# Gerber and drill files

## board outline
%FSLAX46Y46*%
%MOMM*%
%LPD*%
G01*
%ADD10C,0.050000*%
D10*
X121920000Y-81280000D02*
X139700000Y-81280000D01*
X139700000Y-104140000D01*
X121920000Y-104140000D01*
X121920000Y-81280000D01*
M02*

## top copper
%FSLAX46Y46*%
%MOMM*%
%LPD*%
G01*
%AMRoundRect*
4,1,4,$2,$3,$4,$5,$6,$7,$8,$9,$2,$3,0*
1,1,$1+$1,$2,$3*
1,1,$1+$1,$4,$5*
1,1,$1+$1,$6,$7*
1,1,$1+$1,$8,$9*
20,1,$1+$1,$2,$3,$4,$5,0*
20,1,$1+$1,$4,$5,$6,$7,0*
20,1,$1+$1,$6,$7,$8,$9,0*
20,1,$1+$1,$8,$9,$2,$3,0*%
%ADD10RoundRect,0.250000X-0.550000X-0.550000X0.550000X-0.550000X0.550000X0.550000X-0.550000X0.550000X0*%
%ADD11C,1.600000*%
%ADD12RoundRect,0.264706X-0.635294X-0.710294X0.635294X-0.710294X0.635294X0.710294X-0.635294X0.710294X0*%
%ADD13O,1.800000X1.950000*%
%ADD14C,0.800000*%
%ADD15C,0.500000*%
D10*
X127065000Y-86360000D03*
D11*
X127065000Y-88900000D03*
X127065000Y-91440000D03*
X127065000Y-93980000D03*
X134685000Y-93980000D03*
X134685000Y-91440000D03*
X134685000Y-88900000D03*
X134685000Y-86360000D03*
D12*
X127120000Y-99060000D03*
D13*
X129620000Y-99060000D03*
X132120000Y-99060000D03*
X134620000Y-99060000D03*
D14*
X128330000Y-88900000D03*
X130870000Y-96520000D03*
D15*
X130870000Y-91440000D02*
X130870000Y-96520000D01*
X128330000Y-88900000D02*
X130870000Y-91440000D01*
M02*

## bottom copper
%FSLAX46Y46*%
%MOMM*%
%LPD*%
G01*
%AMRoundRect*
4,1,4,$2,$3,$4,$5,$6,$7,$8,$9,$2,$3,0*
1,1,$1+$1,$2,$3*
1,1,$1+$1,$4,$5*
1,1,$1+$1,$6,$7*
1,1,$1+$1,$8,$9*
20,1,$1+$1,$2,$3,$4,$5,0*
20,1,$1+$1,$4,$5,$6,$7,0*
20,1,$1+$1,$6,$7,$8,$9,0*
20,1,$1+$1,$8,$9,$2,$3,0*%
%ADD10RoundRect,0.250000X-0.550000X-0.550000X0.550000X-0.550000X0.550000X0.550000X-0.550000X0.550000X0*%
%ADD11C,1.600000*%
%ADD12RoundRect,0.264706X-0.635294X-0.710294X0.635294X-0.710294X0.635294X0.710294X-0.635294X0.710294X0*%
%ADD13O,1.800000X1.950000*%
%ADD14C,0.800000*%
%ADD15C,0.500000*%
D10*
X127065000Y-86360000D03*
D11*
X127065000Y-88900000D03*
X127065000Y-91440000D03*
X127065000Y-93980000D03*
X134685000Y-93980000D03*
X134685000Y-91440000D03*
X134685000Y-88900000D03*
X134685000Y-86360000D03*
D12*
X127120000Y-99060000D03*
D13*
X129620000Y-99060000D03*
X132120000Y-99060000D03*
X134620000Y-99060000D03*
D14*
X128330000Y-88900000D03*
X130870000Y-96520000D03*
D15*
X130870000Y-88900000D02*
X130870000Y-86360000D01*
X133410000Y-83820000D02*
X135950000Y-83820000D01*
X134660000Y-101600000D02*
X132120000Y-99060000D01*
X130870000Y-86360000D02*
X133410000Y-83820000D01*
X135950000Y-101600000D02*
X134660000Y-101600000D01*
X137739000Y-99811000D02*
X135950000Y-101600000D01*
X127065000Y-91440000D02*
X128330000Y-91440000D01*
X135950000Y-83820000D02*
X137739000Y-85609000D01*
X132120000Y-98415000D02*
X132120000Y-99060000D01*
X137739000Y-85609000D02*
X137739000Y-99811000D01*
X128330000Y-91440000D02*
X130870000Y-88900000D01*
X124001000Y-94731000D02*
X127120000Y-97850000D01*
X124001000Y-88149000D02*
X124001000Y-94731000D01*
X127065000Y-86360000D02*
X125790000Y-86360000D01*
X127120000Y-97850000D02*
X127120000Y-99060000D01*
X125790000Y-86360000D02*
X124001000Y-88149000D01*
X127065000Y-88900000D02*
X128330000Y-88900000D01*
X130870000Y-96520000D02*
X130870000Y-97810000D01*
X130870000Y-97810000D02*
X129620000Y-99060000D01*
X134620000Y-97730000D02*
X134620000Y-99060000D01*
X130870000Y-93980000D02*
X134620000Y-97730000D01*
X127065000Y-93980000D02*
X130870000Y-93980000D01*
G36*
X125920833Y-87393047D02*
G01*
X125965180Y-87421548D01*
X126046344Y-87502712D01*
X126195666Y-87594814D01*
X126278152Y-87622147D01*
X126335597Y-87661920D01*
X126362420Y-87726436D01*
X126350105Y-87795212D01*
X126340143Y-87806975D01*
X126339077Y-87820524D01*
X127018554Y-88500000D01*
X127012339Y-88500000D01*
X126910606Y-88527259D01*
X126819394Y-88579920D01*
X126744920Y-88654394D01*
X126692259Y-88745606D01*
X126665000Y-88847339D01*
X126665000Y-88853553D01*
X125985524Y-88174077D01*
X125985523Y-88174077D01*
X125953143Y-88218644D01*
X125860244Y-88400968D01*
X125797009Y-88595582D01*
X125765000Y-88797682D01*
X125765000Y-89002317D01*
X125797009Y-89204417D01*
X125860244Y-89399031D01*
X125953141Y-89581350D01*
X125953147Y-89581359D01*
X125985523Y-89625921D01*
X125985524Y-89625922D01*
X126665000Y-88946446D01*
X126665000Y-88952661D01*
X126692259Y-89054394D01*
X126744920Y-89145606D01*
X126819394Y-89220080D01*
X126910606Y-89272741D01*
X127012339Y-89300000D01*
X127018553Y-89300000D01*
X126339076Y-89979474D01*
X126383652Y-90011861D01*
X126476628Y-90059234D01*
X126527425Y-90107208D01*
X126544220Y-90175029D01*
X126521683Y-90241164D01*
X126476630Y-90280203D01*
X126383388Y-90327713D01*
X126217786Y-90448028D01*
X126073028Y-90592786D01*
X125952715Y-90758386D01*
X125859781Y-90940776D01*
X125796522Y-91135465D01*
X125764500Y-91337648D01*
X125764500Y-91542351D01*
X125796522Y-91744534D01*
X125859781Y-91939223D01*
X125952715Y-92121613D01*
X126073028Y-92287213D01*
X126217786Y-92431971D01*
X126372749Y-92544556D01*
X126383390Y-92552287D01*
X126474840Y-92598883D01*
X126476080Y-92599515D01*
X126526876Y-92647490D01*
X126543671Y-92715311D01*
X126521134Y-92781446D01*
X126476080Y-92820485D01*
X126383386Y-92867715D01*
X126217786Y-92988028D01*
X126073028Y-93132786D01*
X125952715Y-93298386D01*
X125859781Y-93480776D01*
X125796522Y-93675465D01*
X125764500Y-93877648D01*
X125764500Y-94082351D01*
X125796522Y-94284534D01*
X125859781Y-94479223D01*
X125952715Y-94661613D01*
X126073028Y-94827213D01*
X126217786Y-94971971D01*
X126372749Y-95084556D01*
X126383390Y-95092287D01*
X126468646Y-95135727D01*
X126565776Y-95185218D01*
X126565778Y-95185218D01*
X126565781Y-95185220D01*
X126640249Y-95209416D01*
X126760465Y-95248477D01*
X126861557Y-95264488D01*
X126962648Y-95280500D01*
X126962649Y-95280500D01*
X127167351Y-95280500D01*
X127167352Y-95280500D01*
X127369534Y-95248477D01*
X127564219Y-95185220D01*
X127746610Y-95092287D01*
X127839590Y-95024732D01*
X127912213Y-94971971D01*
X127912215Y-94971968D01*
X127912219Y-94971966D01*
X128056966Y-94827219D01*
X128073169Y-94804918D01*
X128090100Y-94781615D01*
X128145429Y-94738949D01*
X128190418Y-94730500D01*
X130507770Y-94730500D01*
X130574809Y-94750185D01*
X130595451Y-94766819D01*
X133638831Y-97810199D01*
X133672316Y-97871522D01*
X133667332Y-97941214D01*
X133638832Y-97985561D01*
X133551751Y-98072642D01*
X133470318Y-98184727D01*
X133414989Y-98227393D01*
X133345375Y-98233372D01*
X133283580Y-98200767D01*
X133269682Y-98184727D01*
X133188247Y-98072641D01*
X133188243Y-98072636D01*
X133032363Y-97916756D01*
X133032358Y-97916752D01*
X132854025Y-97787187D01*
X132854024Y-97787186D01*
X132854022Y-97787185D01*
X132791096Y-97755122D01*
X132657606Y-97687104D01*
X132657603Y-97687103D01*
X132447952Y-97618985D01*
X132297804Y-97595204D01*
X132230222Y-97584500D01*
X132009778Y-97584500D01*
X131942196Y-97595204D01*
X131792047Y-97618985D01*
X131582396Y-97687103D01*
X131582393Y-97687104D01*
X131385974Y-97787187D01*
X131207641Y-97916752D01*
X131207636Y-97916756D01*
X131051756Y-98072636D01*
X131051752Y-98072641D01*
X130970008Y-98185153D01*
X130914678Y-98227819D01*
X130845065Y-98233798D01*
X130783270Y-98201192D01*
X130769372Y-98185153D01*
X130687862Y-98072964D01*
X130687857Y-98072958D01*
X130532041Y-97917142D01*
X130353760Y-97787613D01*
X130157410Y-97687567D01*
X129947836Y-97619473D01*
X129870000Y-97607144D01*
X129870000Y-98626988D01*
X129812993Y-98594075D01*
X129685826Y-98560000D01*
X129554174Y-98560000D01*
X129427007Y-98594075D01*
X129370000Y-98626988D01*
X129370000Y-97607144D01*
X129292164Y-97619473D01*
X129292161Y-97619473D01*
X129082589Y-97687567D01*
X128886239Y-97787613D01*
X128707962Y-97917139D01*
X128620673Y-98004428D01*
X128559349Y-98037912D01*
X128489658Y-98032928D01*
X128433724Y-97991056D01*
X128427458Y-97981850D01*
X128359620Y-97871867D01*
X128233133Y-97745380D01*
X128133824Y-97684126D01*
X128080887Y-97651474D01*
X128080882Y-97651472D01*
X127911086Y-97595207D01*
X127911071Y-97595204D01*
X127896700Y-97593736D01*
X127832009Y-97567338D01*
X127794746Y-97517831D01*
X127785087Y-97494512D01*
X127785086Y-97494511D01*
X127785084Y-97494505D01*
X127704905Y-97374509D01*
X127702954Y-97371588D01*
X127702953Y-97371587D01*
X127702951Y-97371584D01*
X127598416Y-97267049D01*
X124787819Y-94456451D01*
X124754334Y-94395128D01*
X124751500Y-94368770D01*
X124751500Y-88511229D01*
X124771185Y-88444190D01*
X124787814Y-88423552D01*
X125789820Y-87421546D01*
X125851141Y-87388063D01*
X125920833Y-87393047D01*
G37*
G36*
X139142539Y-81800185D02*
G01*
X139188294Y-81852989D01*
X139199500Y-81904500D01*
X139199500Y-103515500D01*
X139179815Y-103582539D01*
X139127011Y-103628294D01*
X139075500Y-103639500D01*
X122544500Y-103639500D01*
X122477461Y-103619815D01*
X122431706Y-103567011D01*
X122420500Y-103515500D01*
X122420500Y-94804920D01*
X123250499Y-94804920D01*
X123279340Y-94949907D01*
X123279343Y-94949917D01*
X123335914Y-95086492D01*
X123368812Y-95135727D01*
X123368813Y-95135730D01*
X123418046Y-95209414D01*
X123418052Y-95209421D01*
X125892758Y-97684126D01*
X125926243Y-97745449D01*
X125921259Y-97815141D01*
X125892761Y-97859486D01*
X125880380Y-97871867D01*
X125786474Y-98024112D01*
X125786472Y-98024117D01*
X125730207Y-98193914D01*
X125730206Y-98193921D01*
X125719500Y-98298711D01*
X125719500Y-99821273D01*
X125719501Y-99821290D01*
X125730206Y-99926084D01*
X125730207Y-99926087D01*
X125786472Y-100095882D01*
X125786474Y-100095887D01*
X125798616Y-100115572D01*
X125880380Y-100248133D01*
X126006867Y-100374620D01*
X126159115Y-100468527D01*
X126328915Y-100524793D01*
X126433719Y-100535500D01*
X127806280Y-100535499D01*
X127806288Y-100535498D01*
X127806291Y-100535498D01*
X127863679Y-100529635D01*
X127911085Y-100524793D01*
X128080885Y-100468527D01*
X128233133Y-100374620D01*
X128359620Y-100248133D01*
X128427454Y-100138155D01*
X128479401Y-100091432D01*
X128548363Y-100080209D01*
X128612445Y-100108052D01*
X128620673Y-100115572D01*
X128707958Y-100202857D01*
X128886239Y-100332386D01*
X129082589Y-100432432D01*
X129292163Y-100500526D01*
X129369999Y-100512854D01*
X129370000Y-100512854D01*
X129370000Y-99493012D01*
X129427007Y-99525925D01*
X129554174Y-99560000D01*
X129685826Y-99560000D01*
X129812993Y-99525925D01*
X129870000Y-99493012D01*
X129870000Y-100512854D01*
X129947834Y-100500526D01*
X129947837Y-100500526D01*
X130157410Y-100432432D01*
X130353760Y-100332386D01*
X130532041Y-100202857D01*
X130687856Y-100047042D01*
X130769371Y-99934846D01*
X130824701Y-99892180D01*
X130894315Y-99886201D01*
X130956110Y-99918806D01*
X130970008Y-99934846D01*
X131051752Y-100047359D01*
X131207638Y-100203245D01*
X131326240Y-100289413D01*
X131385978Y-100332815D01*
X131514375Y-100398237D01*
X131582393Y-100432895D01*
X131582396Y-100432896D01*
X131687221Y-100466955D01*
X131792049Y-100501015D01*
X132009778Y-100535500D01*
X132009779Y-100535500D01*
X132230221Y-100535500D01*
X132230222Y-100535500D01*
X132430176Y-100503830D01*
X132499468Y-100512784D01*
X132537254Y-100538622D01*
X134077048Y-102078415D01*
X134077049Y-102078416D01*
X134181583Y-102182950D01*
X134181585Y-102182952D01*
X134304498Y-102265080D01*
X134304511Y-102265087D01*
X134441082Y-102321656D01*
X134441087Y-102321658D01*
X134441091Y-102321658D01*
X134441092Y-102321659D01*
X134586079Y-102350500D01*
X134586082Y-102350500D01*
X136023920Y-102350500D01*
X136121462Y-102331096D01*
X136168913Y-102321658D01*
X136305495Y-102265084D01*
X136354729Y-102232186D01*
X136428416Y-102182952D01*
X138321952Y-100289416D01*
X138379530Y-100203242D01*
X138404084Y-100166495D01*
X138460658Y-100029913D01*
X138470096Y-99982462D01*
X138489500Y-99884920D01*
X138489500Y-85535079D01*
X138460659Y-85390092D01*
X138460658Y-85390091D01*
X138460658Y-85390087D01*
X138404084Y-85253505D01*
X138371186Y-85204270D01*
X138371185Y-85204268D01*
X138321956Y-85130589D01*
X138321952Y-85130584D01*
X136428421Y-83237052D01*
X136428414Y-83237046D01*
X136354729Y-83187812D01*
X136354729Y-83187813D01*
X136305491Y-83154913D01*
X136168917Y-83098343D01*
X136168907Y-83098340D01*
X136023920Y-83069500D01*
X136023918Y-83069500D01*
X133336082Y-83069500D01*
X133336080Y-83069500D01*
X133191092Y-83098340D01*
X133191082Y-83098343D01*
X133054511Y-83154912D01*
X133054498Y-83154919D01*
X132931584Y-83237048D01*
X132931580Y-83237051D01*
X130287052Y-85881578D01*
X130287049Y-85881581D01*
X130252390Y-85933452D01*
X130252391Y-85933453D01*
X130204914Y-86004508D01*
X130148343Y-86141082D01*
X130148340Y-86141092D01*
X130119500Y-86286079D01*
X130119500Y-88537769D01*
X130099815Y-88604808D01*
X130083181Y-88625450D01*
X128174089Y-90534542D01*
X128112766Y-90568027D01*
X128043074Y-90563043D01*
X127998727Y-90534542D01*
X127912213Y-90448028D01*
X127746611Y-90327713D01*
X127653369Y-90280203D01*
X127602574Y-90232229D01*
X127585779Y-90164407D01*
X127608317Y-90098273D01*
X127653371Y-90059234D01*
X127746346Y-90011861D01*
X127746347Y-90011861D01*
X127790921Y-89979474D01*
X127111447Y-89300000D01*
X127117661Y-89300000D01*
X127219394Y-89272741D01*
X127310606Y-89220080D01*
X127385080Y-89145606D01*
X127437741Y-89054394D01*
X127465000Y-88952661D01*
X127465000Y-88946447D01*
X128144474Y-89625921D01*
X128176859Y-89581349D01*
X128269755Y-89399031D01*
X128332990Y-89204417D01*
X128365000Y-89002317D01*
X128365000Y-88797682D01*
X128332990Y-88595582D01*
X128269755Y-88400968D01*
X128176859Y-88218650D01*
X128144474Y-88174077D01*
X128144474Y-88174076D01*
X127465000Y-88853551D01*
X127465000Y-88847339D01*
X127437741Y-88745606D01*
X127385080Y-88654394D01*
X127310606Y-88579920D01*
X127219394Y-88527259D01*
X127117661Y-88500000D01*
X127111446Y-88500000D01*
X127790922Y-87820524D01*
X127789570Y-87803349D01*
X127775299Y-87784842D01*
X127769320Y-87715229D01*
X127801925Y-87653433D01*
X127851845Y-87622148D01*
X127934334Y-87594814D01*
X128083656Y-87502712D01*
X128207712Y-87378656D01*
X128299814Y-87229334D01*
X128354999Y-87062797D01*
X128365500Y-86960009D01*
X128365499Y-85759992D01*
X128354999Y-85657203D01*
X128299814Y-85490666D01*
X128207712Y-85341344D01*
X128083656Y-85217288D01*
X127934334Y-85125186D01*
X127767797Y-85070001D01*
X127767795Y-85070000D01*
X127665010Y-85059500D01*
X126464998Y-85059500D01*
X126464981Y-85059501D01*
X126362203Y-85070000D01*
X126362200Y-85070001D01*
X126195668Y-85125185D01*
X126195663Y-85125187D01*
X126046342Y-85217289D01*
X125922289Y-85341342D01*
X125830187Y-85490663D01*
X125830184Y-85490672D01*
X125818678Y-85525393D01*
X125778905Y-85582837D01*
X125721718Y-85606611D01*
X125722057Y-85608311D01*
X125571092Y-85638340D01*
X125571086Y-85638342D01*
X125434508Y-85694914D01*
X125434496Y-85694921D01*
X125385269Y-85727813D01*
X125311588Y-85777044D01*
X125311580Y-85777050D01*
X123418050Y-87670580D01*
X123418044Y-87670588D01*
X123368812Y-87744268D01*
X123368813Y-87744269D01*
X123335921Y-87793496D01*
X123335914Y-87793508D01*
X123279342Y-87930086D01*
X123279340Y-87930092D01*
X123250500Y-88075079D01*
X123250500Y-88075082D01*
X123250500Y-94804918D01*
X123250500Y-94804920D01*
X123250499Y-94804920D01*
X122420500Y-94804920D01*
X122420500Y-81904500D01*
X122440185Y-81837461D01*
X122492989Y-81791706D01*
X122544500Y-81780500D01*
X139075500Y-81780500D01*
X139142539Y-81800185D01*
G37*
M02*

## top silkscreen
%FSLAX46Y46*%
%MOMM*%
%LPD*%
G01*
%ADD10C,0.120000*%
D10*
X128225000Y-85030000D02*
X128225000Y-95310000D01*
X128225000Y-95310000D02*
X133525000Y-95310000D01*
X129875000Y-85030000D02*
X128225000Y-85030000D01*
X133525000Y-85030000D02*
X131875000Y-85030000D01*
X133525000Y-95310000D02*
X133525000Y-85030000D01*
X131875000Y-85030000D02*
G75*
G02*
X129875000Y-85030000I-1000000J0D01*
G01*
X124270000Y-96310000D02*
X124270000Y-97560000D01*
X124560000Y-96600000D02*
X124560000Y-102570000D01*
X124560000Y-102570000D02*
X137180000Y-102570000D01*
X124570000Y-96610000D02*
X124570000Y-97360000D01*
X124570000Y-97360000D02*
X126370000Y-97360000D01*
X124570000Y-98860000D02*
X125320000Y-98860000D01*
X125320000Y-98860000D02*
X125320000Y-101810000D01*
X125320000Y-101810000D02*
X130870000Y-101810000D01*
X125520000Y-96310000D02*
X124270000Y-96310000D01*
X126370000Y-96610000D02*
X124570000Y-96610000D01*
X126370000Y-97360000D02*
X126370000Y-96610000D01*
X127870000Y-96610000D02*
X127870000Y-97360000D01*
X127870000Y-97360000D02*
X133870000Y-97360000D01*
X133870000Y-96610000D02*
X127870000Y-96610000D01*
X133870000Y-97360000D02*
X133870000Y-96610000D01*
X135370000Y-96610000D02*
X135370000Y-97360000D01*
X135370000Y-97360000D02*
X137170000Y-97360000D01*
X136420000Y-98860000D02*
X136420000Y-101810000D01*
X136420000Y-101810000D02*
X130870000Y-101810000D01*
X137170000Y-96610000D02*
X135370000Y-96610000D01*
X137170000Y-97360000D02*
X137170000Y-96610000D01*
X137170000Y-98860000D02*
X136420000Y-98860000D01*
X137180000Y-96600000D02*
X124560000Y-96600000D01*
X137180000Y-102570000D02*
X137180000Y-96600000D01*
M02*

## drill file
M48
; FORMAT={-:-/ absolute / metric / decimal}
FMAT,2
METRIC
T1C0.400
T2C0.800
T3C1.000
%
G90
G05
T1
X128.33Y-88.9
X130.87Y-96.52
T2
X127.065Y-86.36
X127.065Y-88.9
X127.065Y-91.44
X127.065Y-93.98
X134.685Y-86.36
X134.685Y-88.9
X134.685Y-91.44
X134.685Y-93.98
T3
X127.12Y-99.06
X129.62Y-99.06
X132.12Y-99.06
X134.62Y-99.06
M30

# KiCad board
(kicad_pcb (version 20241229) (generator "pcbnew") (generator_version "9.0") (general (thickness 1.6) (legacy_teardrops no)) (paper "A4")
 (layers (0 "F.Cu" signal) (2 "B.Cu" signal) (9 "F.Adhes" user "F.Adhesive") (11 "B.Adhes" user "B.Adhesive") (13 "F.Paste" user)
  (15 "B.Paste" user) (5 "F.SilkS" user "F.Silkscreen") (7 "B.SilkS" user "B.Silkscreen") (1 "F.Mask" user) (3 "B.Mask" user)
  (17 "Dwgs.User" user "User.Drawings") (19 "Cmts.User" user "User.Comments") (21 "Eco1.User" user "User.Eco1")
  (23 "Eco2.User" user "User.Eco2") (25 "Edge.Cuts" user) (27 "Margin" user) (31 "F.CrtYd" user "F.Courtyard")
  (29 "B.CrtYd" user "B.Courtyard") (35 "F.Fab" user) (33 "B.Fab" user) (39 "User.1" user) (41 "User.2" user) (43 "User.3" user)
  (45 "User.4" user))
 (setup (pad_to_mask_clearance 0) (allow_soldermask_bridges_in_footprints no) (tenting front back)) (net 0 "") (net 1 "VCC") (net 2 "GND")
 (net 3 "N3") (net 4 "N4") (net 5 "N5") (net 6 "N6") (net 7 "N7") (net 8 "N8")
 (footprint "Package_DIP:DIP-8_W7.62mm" (layer "F.Cu") (at 127.065 86.36)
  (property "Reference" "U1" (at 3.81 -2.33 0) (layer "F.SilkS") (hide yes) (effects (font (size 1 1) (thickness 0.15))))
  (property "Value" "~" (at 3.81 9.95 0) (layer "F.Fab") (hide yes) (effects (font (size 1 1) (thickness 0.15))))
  (fp_line (start 1.16 -1.33) (end 1.16 8.95) (stroke (width 0.12) (type solid)) (layer "F.SilkS"))
  (fp_line (start 1.16 8.95) (end 6.46 8.95) (stroke (width 0.12) (type solid)) (layer "F.SilkS"))
  (fp_line (start 2.81 -1.33) (end 1.16 -1.33) (stroke (width 0.12) (type solid)) (layer "F.SilkS"))
  (fp_line (start 6.46 -1.33) (end 4.81 -1.33) (stroke (width 0.12) (type solid)) (layer "F.SilkS"))
  (fp_line (start 6.46 8.95) (end 6.46 -1.33) (stroke (width 0.12) (type solid)) (layer "F.SilkS"))
  (fp_arc (start 4.81 -1.33) (mid 3.81 -0.33) (end 2.81 -1.33) (stroke (width 0.12) (type solid)) (layer "F.SilkS"))
  (pad "1" thru_hole roundrect (at 0 0) (size 1.6 1.6) (drill 0.8) (layers "*.Cu" "*.Mask") (remove_unused_layers no)
   (roundrect_rratio 0.15625) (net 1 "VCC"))
  (pad "2" thru_hole circle (at 0 2.54) (size 1.6 1.6) (drill 0.8) (layers "*.Cu" "*.Mask") (remove_unused_layers no) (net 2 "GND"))
  (pad "3" thru_hole circle (at 0 5.08) (size 1.6 1.6) (drill 0.8) (layers "*.Cu" "*.Mask") (remove_unused_layers no) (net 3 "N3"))
  (pad "4" thru_hole circle (at 0 7.62) (size 1.6 1.6) (drill 0.8) (layers "*.Cu" "*.Mask") (remove_unused_layers no) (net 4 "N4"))
  (pad "5" thru_hole circle (at 7.62 7.62) (size 1.6 1.6) (drill 0.8) (layers "*.Cu" "*.Mask") (remove_unused_layers no) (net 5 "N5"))
  (pad "6" thru_hole circle (at 7.62 5.08) (size 1.6 1.6) (drill 0.8) (layers "*.Cu" "*.Mask") (remove_unused_layers no) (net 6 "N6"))
  (pad "7" thru_hole circle (at 7.62 2.54) (size 1.6 1.6) (drill 0.8) (layers "*.Cu" "*.Mask") (remove_unused_layers no) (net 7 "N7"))
  (pad "8" thru_hole circle (at 7.62 0) (size 1.6 1.6) (drill 0.8) (layers "*.Cu" "*.Mask") (remove_unused_layers no) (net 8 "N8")))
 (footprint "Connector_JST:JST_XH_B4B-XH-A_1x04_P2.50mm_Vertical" (layer "F.Cu") (at 127.12 99.06)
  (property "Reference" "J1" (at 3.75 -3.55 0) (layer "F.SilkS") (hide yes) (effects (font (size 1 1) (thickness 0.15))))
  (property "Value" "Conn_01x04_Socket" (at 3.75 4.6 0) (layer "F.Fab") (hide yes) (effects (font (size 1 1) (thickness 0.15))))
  (fp_line (start -2.85 -2.75) (end -2.85 -1.5) (stroke (width 0.12) (type solid)) (layer "F.SilkS"))
  (fp_line (start -2.56 -2.46) (end -2.56 3.51) (stroke (width 0.12) (type solid)) (layer "F.SilkS"))
  (fp_line (start -2.56 3.51) (end 10.06 3.51) (stroke (width 0.12) (type solid)) (layer "F.SilkS"))
  (fp_line (start -2.55 -2.45) (end -2.55 -1.7) (stroke (width 0.12) (type solid)) (layer "F.SilkS"))
  (fp_line (start -2.55 -1.7) (end -0.75 -1.7) (stroke (width 0.12) (type solid)) (layer "F.SilkS"))
  (fp_line (start -2.55 -0.2) (end -1.8 -0.2) (stroke (width 0.12) (type solid)) (layer "F.SilkS"))
  (fp_line (start -1.8 -0.2) (end -1.8 2.75) (stroke (width 0.12) (type solid)) (layer "F.SilkS"))
  (fp_line (start -1.8 2.75) (end 3.75 2.75) (stroke (width 0.12) (type solid)) (layer "F.SilkS"))
  (fp_line (start -1.6 -2.75) (end -2.85 -2.75) (stroke (width 0.12) (type solid)) (layer "F.SilkS"))
  (fp_line (start -0.75 -2.45) (end -2.55 -2.45) (stroke (width 0.12) (type solid)) (layer "F.SilkS"))
  (fp_line (start -0.75 -1.7) (end -0.75 -2.45) (stroke (width 0.12) (type solid)) (layer "F.SilkS"))
  (fp_line (start 0.75 -2.45) (end 0.75 -1.7) (stroke (width 0.12) (type solid)) (layer "F.SilkS"))
  (fp_line (start 0.75 -1.7) (end 6.75 -1.7) (stroke (width 0.12) (type solid)) (layer "F.SilkS"))
  (fp_line (start 6.75 -2.45) (end 0.75 -2.45) (stroke (width 0.12) (type solid)) (layer "F.SilkS"))
  (fp_line (start 6.75 -1.7) (end 6.75 -2.45) (stroke (width 0.12) (type solid)) (layer "F.SilkS"))
  (fp_line (start 8.25 -2.45) (end 8.25 -1.7) (stroke (width 0.12) (type solid)) (layer "F.SilkS"))
  (fp_line (start 8.25 -1.7) (end 10.05 -1.7) (stroke (width 0.12) (type solid)) (layer "F.SilkS"))
  (fp_line (start 9.3 -0.2) (end 9.3 2.75) (stroke (width 0.12) (type solid)) (layer "F.SilkS"))
  (fp_line (start 9.3 2.75) (end 3.75 2.75) (stroke (width 0.12) (type solid)) (layer "F.SilkS"))
  (fp_line (start 10.05 -2.45) (end 8.25 -2.45) (stroke (width 0.12) (type solid)) (layer "F.SilkS"))
  (fp_line (start 10.05 -1.7) (end 10.05 -2.45) (stroke (width 0.12) (type solid)) (layer "F.SilkS"))
  (fp_line (start 10.05 -0.2) (end 9.3 -0.2) (stroke (width 0.12) (type solid)) (layer "F.SilkS"))
  (fp_line (start 10.06 -2.46) (end -2.56 -2.46) (stroke (width 0.12) (type solid)) (layer "F.SilkS"))
  (fp_line (start 10.06 3.51) (end 10.06 -2.46) (stroke (width 0.12) (type solid)) (layer "F.SilkS"))
  (pad "1" thru_hole roundrect (at 0 0) (size 1.8 1.95) (drill 1) (layers "*.Cu" "*.Mask") (remove_unused_layers no)
   (roundrect_rratio 0.147059) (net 1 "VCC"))
  (pad "2" thru_hole oval (at 2.5 0) (size 1.8 1.95) (drill 1) (layers "*.Cu" "*.Mask") (remove_unused_layers no) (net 2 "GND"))
  (pad "3" thru_hole oval (at 5 0) (size 1.8 1.95) (drill 1) (layers "*.Cu" "*.Mask") (remove_unused_layers no) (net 3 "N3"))
  (pad "4" thru_hole oval (at 7.5 0) (size 1.8 1.95) (drill 1) (layers "*.Cu" "*.Mask") (remove_unused_layers no) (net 4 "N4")))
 (gr_rect (start 121.92 81.28) (end 139.7 104.14) (stroke (width 0.05) (type default)) (fill no) (layer "Edge.Cuts"))
 (segment (start 130.87 88.9) (end 130.87 86.36) (width 0.5) (layer "B.Cu") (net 3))
 (segment (start 133.41 83.82) (end 135.95 83.82) (width 0.5) (layer "B.Cu") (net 3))
 (segment (start 134.66 101.6) (end 132.12 99.06) (width 0.5) (layer "B.Cu") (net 3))
 (segment (start 130.87 86.36) (end 133.41 83.82) (width 0.5) (layer "B.Cu") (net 3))
 (segment (start 135.95 101.6) (end 134.66 101.6) (width 0.5) (layer "B.Cu") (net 3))
 (segment (start 137.739 99.811) (end 135.95 101.6) (width 0.5) (layer "B.Cu") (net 3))
 (segment (start 127.065 91.44) (end 128.33 91.44) (width 0.5) (layer "B.Cu") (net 3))
 (segment (start 135.95 83.82) (end 137.739 85.609) (width 0.5) (layer "B.Cu") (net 3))
 (segment (start 132.12 98.415) (end 132.12 99.06) (width 0.5) (layer "B.Cu") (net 3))
 (segment (start 137.739 85.609) (end 137.739 99.811) (width 0.5) (layer "B.Cu") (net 3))
 (segment (start 128.33 91.44) (end 130.87 88.9) (width 0.5) (layer "B.Cu") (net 3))
 (segment (start 124.001 94.731) (end 127.12 97.85) (width 0.5) (layer "B.Cu") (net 1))
 (segment (start 124.001 88.149) (end 124.001 94.731) (width 0.5) (layer "B.Cu") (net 1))
 (segment (start 127.065 86.36) (end 125.79 86.36) (width 0.5) (layer "B.Cu") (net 1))
 (segment (start 127.12 97.85) (end 127.12 99.06) (width 0.5) (layer "B.Cu") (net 1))
 (segment (start 125.79 86.36) (end 124.001 88.149) (width 0.5) (layer "B.Cu") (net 1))
 (segment (start 130.87 91.44) (end 130.87 96.52) (width 0.5) (layer "F.Cu") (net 2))
 (segment (start 128.33 88.9) (end 130.87 91.44) (width 0.5) (layer "F.Cu") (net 2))
 (via (at 128.33 88.9) (size 0.8) (drill 0.4) (layers "F.Cu" "B.Cu") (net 2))
 (via (at 130.87 96.52) (size 0.8) (drill 0.4) (layers "F.Cu" "B.Cu") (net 2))
 (segment (start 127.065 88.9) (end 128.33 88.9) (width 0.5) (layer "B.Cu") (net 2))
 (segment (start 130.87 96.52) (end 130.87 97.81) (width 0.5) (layer "B.Cu") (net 2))
 (segment (start 130.87 97.81) (end 129.62 99.06) (width 0.5) (layer "B.Cu") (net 2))
 (segment (start 134.62 97.73) (end 134.62 99.06) (width 0.5) (layer "B.Cu") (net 4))
 (segment (start 130.87 93.98) (end 134.62 97.73) (width 0.5) (layer "B.Cu") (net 4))
 (segment (start 127.065 93.98) (end 130.87 93.98) (width 0.5) (layer "B.Cu") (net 4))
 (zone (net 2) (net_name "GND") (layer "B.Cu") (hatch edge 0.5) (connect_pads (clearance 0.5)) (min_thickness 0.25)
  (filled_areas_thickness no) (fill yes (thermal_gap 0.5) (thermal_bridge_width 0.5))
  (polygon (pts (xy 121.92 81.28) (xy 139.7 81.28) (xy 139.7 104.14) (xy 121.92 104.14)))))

